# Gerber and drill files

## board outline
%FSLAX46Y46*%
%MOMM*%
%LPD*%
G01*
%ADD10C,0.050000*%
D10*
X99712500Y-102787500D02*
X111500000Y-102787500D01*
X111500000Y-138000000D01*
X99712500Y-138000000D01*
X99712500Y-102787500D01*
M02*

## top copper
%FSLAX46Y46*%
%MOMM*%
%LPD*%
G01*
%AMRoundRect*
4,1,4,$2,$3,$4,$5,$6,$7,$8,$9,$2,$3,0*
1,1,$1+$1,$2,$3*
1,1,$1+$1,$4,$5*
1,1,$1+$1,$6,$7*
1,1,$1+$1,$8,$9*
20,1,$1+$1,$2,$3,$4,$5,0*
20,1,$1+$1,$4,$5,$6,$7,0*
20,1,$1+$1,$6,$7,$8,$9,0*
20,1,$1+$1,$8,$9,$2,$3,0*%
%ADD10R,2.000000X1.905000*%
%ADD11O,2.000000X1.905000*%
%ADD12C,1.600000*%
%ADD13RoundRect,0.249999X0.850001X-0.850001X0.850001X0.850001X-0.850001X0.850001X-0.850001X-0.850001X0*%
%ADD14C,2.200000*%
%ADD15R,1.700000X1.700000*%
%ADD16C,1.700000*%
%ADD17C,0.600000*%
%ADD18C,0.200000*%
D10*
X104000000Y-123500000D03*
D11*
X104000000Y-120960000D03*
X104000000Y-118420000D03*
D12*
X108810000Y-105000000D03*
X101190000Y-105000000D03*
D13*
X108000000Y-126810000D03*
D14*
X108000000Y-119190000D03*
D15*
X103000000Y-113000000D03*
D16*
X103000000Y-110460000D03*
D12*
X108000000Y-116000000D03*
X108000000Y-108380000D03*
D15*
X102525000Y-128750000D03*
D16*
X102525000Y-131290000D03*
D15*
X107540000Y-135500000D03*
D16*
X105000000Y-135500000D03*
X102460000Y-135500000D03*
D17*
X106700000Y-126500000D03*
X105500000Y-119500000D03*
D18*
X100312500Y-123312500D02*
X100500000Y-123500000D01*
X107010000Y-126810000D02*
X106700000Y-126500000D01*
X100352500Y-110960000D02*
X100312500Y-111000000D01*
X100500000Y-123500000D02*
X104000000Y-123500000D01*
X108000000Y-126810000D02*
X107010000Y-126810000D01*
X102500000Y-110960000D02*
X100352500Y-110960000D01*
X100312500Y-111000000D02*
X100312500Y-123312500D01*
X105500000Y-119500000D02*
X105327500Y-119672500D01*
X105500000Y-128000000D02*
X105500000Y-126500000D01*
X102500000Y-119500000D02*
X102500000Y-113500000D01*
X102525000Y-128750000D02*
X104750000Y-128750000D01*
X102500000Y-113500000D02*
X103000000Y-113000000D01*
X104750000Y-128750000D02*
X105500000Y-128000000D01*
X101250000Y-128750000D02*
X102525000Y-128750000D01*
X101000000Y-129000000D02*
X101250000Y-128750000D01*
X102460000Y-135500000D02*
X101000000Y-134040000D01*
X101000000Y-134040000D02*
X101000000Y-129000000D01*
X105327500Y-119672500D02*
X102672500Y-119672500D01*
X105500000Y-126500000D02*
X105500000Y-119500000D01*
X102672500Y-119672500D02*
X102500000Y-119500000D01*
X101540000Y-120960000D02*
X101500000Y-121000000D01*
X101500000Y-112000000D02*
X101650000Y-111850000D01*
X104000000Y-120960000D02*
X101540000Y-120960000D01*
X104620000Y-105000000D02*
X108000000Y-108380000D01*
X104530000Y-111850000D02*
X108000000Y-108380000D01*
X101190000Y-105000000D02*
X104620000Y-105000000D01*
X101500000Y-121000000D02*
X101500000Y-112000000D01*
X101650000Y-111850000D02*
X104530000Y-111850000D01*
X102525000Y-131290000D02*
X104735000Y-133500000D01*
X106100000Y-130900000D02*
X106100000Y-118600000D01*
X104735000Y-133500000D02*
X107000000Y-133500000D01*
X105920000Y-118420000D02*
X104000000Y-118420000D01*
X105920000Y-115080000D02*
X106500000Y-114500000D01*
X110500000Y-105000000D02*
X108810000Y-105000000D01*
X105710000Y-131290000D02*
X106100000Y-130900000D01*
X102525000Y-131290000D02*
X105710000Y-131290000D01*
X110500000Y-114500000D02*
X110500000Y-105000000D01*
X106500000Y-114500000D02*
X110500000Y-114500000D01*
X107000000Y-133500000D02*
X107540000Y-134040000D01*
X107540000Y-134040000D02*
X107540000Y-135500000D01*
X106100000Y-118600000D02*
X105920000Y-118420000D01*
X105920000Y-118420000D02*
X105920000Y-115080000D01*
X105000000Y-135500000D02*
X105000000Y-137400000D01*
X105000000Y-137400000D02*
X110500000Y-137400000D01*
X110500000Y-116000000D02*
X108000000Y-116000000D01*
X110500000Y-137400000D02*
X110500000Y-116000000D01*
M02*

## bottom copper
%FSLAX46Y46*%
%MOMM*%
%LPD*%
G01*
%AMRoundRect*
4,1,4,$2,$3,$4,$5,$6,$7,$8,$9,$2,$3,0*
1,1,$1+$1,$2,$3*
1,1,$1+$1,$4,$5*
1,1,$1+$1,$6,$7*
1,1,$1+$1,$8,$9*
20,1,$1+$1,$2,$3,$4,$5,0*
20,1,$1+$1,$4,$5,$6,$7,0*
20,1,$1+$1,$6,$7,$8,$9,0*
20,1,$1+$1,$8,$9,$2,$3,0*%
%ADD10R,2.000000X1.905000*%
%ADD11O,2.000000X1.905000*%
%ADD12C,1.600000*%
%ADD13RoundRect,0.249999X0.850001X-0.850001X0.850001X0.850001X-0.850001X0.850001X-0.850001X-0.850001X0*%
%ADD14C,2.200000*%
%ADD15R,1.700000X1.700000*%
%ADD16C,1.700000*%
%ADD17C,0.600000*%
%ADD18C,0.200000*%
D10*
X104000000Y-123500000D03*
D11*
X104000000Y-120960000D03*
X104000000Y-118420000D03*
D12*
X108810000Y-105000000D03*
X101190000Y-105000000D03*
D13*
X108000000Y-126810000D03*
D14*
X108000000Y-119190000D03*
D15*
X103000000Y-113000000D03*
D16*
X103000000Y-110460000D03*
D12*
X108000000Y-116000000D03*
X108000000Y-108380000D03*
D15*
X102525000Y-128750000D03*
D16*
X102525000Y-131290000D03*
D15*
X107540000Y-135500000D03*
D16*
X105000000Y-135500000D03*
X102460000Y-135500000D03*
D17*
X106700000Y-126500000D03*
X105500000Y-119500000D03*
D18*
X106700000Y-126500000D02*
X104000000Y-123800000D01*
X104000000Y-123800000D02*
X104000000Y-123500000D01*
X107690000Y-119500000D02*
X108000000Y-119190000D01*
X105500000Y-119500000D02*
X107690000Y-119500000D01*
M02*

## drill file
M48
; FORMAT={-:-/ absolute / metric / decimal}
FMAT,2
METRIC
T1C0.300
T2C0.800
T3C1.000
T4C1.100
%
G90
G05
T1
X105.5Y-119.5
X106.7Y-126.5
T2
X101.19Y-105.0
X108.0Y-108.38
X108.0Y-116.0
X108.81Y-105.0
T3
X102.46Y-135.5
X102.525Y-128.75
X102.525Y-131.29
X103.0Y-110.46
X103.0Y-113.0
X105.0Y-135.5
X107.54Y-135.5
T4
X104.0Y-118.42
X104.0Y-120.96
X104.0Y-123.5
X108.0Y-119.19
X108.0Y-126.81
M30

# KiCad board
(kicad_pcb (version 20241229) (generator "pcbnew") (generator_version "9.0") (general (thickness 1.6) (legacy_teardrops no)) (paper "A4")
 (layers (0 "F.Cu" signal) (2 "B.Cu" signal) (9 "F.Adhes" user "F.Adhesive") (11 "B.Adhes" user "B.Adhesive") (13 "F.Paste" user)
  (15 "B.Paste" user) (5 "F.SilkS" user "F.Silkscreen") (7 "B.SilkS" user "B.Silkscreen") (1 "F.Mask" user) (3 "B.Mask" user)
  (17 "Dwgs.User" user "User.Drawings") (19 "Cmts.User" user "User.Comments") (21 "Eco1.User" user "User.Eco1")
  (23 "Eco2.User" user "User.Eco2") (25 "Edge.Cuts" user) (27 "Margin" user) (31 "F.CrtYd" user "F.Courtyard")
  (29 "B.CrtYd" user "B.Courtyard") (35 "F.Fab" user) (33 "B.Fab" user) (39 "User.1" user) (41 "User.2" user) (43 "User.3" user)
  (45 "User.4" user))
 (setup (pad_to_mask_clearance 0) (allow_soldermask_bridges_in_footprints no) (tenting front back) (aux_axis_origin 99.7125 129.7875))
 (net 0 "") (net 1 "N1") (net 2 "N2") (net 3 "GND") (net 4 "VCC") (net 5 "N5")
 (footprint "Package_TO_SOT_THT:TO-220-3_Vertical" (layer "F.Cu") (at 104 123.5 90)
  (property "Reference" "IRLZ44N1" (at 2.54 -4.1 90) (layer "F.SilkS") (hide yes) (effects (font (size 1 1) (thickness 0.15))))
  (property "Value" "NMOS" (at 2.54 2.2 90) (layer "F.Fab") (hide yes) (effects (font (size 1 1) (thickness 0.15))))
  (pad "1" thru_hole rect (at 0 0 90) (size 1.905 2) (drill 1.1) (layers "*.Cu" "*.Mask") (remove_unused_layers no) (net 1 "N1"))
  (pad "2" thru_hole oval (at 2.54 0 90) (size 1.905 2) (drill 1.1) (layers "*.Cu" "*.Mask") (remove_unused_layers no) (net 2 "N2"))
  (pad "3" thru_hole oval (at 5.08 0 90) (size 1.905 2) (drill 1.1) (layers "*.Cu" "*.Mask") (remove_unused_layers no) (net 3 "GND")))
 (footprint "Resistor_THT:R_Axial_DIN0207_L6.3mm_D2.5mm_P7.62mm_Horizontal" (layer "F.Cu") (at 108.81 105 180)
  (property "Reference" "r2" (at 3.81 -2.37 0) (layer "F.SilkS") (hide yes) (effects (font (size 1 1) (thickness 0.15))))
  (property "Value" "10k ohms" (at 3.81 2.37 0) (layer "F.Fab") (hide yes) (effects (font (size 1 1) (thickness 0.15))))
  (pad "1" thru_hole circle (at 0 0 180) (size 1.6 1.6) (drill 0.8) (layers "*.Cu" "*.Mask") (remove_unused_layers no) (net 3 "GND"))
  (pad "2" thru_hole circle (at 7.62 0 180) (size 1.6 1.6) (drill 0.8) (layers "*.Cu" "*.Mask") (remove_unused_layers no) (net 2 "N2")))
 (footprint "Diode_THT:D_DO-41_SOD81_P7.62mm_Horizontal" (layer "F.Cu") (at 108 126.81 90)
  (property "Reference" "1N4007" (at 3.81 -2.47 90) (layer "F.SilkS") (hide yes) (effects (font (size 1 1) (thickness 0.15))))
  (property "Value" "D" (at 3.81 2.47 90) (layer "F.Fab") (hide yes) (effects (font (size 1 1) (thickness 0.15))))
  (pad "1" thru_hole roundrect (at 0 0 90) (size 2.2 2.2) (drill 1.1) (layers "*.Cu" "*.Mask") (remove_unused_layers no)
   (roundrect_rratio 0.113636) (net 1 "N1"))
  (pad "2" thru_hole circle (at 7.62 0 90) (size 2.2 2.2) (drill 1.1) (layers "*.Cu" "*.Mask") (remove_unused_layers no) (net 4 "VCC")))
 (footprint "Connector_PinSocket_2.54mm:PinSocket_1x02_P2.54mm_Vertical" (layer "F.Cu") (at 103 113 180)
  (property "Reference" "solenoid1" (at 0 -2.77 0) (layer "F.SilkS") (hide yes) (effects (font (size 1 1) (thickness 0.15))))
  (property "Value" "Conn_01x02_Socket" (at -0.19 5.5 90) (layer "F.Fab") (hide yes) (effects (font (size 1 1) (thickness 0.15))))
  (pad "1" thru_hole rect (at 0 0 180) (size 1.7 1.7) (drill 1) (layers "*.Cu" "*.Mask") (remove_unused_layers no) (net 4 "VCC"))
  (pad "2" thru_hole circle (at 0 2.54 180) (size 1.7 1.7) (drill 1) (layers "*.Cu" "*.Mask") (remove_unused_layers no) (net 1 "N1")))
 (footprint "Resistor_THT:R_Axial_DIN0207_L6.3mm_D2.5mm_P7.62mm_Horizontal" (layer "F.Cu") (at 108 116 90)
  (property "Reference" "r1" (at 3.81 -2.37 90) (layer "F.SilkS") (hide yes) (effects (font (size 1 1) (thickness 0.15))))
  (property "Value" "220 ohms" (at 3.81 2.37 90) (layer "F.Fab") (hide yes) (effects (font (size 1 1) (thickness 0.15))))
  (pad "1" thru_hole circle (at 0 0 90) (size 1.6 1.6) (drill 0.8) (layers "*.Cu" "*.Mask") (remove_unused_layers no) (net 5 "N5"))
  (pad "2" thru_hole circle (at 7.62 0 90) (size 1.6 1.6) (drill 0.8) (layers "*.Cu" "*.Mask") (remove_unused_layers no) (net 2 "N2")))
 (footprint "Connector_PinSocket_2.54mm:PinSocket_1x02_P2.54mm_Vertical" (layer "F.Cu") (at 102.525 128.75)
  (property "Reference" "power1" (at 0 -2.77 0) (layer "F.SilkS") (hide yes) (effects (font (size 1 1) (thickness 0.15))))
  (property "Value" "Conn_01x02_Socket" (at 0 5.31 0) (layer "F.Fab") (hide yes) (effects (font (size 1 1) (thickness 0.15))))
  (pad "1" thru_hole rect (at 0 0) (size 1.7 1.7) (drill 1) (layers "*.Cu" "*.Mask") (remove_unused_layers no) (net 4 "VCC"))
  (pad "2" thru_hole circle (at 0 2.54) (size 1.7 1.7) (drill 1) (layers "*.Cu" "*.Mask") (remove_unused_layers no) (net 3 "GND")))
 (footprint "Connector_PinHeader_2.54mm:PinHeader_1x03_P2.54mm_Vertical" (layer "F.Cu") (at 107.54 135.5 -90)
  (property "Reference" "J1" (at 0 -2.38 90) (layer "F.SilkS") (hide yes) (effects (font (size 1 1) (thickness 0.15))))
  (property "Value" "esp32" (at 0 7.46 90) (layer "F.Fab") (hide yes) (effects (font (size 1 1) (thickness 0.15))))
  (pad "1" thru_hole rect (at 0 0 270) (size 1.7 1.7) (drill 1) (layers "*.Cu" "*.Mask") (remove_unused_layers no) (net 3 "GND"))
  (pad "2" thru_hole circle (at 0 2.54 270) (size 1.7 1.7) (drill 1) (layers "*.Cu" "*.Mask") (remove_unused_layers no) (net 5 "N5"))
  (pad "3" thru_hole circle (at 0 5.08 270) (size 1.7 1.7) (drill 1) (layers "*.Cu" "*.Mask") (remove_unused_layers no) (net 4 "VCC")))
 (gr_rect (start 99.7125 102.7875) (end 111.5 138) (stroke (width 0.05) (type default)) (fill no) (layer "Edge.Cuts"))
 (segment (start 100.3125 123.3125) (end 100.5 123.5) (width 0.2) (layer "F.Cu") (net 1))
 (segment (start 107.01 126.81) (end 106.7 126.5) (width 0.2) (layer "F.Cu") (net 1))
 (segment (start 100.3525 110.96) (end 100.3125 111) (width 0.2) (layer "F.Cu") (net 1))
 (segment (start 100.5 123.5) (end 104 123.5) (width 0.2) (layer "F.Cu") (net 1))
 (segment (start 108 126.81) (end 107.01 126.81) (width 0.2) (layer "F.Cu") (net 1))
 (segment (start 102.5 110.96) (end 100.3525 110.96) (width 0.2) (layer "F.Cu") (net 1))
 (segment (start 100.3125 111) (end 100.3125 123.3125) (width 0.2) (layer "F.Cu") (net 1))
 (via (at 106.7 126.5) (size 0.6) (drill 0.3) (layers "F.Cu" "B.Cu") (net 1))
 (segment (start 106.7 126.5) (end 104 123.8) (width 0.2) (layer "B.Cu") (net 1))
 (segment (start 104 123.8) (end 104 123.5) (width 0.2) (layer "B.Cu") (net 1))
 (segment (start 105.5 119.5) (end 105.3275 119.6725) (width 0.2) (layer "F.Cu") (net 4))
 (segment (start 105.5 128) (end 105.5 126.5) (width 0.2) (layer "F.Cu") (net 4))
 (segment (start 102.5 119.5) (end 102.5 113.5) (width 0.2) (layer "F.Cu") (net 4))
 (segment (start 102.525 128.75) (end 104.75 128.75) (width 0.2) (layer "F.Cu") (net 4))
 (segment (start 102.5 113.5) (end 103 113) (width 0.2) (layer "F.Cu") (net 4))
 (segment (start 104.75 128.75) (end 105.5 128) (width 0.2) (layer "F.Cu") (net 4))
 (segment (start 101.25 128.75) (end 102.525 128.75) (width 0.2) (layer "F.Cu") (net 4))
 (segment (start 101 129) (end 101.25 128.75) (width 0.2) (layer "F.Cu") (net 4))
 (segment (start 102.46 135.5) (end 101 134.04) (width 0.2) (layer "F.Cu") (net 4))
 (segment (start 101 134.04) (end 101 129) (width 0.2) (layer "F.Cu") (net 4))
 (segment (start 105.3275 119.6725) (end 102.6725 119.6725) (width 0.2) (layer "F.Cu") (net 4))
 (segment (start 105.5 126.5) (end 105.5 119.5) (width 0.2) (layer "F.Cu") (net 4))
 (segment (start 102.6725 119.6725) (end 102.5 119.5) (width 0.2) (layer "F.Cu") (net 4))
 (via (at 105.5 119.5) (size 0.6) (drill 0.3) (layers "F.Cu" "B.Cu") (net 4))
 (segment (start 107.69 119.5) (end 108 119.19) (width 0.2) (layer "B.Cu") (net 4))
 (segment (start 105.5 119.5) (end 107.69 119.5) (width 0.2) (layer "B.Cu") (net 4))
 (segment (start 101.54 120.96) (end 101.5 121) (width 0.2) (layer "F.Cu") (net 2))
 (segment (start 101.5 112) (end 101.65 111.85) (width 0.2) (layer "F.Cu") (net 2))
 (segment (start 104 120.96) (end 101.54 120.96) (width 0.2) (layer "F.Cu") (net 2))
 (segment (start 104.62 105) (end 108 108.38) (width 0.2) (layer "F.Cu") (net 2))
 (segment (start 104.53 111.85) (end 108 108.38) (width 0.2) (layer "F.Cu") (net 2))
 (segment (start 101.19 105) (end 104.62 105) (width 0.2) (layer "F.Cu") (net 2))
 (segment (start 101.5 121) (end 101.5 112) (width 0.2) (layer "F.Cu") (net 2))
 (segment (start 101.65 111.85) (end 104.53 111.85) (width 0.2) (layer "F.Cu") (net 2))
 (segment (start 102.525 131.29) (end 104.735 133.5) (width 0.2) (layer "F.Cu") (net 3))
 (segment (start 106.1 130.9) (end 106.1 118.6) (width 0.2) (layer "F.Cu") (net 3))
 (segment (start 104.735 133.5) (end 107 133.5) (width 0.2) (layer "F.Cu") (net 3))
 (segment (start 105.92 118.42) (end 104 118.42) (width 0.2) (layer "F.Cu") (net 3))
 (segment (start 105.92 115.08) (end 106.5 114.5) (width 0.2) (layer "F.Cu") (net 3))
 (segment (start 110.5 105) (end 108.81 105) (width 0.2) (layer "F.Cu") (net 3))
 (segment (start 105.71 131.29) (end 106.1 130.9) (width 0.2) (layer "F.Cu") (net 3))
 (segment (start 102.525 131.29) (end 105.71 131.29) (width 0.2) (layer "F.Cu") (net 3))
 (segment (start 110.5 114.5) (end 110.5 105) (width 0.2) (layer "F.Cu") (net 3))
 (segment (start 106.5 114.5) (end 110.5 114.5) (width 0.2) (layer "F.Cu") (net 3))
 (segment (start 107 133.5) (end 107.54 134.04) (width 0.2) (layer "F.Cu") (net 3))
 (segment (start 107.54 134.04) (end 107.54 135.5) (width 0.2) (layer "F.Cu") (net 3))
 (segment (start 106.1 118.6) (end 105.92 118.42) (width 0.2) (layer "F.Cu") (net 3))
 (segment (start 105.92 118.42) (end 105.92 115.08) (width 0.2) (layer "F.Cu") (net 3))
 (segment (start 105 135.5) (end 105 137.4) (width 0.2) (layer "F.Cu") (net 5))
 (segment (start 105 137.4) (end 110.5 137.4) (width 0.2) (layer "F.Cu") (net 5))
 (segment (start 110.5 116) (end 108 116) (width 0.2) (layer "F.Cu") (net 5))
 (segment (start 110.5 137.4) (end 110.5 116) (width 0.2) (layer "F.Cu") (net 5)))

